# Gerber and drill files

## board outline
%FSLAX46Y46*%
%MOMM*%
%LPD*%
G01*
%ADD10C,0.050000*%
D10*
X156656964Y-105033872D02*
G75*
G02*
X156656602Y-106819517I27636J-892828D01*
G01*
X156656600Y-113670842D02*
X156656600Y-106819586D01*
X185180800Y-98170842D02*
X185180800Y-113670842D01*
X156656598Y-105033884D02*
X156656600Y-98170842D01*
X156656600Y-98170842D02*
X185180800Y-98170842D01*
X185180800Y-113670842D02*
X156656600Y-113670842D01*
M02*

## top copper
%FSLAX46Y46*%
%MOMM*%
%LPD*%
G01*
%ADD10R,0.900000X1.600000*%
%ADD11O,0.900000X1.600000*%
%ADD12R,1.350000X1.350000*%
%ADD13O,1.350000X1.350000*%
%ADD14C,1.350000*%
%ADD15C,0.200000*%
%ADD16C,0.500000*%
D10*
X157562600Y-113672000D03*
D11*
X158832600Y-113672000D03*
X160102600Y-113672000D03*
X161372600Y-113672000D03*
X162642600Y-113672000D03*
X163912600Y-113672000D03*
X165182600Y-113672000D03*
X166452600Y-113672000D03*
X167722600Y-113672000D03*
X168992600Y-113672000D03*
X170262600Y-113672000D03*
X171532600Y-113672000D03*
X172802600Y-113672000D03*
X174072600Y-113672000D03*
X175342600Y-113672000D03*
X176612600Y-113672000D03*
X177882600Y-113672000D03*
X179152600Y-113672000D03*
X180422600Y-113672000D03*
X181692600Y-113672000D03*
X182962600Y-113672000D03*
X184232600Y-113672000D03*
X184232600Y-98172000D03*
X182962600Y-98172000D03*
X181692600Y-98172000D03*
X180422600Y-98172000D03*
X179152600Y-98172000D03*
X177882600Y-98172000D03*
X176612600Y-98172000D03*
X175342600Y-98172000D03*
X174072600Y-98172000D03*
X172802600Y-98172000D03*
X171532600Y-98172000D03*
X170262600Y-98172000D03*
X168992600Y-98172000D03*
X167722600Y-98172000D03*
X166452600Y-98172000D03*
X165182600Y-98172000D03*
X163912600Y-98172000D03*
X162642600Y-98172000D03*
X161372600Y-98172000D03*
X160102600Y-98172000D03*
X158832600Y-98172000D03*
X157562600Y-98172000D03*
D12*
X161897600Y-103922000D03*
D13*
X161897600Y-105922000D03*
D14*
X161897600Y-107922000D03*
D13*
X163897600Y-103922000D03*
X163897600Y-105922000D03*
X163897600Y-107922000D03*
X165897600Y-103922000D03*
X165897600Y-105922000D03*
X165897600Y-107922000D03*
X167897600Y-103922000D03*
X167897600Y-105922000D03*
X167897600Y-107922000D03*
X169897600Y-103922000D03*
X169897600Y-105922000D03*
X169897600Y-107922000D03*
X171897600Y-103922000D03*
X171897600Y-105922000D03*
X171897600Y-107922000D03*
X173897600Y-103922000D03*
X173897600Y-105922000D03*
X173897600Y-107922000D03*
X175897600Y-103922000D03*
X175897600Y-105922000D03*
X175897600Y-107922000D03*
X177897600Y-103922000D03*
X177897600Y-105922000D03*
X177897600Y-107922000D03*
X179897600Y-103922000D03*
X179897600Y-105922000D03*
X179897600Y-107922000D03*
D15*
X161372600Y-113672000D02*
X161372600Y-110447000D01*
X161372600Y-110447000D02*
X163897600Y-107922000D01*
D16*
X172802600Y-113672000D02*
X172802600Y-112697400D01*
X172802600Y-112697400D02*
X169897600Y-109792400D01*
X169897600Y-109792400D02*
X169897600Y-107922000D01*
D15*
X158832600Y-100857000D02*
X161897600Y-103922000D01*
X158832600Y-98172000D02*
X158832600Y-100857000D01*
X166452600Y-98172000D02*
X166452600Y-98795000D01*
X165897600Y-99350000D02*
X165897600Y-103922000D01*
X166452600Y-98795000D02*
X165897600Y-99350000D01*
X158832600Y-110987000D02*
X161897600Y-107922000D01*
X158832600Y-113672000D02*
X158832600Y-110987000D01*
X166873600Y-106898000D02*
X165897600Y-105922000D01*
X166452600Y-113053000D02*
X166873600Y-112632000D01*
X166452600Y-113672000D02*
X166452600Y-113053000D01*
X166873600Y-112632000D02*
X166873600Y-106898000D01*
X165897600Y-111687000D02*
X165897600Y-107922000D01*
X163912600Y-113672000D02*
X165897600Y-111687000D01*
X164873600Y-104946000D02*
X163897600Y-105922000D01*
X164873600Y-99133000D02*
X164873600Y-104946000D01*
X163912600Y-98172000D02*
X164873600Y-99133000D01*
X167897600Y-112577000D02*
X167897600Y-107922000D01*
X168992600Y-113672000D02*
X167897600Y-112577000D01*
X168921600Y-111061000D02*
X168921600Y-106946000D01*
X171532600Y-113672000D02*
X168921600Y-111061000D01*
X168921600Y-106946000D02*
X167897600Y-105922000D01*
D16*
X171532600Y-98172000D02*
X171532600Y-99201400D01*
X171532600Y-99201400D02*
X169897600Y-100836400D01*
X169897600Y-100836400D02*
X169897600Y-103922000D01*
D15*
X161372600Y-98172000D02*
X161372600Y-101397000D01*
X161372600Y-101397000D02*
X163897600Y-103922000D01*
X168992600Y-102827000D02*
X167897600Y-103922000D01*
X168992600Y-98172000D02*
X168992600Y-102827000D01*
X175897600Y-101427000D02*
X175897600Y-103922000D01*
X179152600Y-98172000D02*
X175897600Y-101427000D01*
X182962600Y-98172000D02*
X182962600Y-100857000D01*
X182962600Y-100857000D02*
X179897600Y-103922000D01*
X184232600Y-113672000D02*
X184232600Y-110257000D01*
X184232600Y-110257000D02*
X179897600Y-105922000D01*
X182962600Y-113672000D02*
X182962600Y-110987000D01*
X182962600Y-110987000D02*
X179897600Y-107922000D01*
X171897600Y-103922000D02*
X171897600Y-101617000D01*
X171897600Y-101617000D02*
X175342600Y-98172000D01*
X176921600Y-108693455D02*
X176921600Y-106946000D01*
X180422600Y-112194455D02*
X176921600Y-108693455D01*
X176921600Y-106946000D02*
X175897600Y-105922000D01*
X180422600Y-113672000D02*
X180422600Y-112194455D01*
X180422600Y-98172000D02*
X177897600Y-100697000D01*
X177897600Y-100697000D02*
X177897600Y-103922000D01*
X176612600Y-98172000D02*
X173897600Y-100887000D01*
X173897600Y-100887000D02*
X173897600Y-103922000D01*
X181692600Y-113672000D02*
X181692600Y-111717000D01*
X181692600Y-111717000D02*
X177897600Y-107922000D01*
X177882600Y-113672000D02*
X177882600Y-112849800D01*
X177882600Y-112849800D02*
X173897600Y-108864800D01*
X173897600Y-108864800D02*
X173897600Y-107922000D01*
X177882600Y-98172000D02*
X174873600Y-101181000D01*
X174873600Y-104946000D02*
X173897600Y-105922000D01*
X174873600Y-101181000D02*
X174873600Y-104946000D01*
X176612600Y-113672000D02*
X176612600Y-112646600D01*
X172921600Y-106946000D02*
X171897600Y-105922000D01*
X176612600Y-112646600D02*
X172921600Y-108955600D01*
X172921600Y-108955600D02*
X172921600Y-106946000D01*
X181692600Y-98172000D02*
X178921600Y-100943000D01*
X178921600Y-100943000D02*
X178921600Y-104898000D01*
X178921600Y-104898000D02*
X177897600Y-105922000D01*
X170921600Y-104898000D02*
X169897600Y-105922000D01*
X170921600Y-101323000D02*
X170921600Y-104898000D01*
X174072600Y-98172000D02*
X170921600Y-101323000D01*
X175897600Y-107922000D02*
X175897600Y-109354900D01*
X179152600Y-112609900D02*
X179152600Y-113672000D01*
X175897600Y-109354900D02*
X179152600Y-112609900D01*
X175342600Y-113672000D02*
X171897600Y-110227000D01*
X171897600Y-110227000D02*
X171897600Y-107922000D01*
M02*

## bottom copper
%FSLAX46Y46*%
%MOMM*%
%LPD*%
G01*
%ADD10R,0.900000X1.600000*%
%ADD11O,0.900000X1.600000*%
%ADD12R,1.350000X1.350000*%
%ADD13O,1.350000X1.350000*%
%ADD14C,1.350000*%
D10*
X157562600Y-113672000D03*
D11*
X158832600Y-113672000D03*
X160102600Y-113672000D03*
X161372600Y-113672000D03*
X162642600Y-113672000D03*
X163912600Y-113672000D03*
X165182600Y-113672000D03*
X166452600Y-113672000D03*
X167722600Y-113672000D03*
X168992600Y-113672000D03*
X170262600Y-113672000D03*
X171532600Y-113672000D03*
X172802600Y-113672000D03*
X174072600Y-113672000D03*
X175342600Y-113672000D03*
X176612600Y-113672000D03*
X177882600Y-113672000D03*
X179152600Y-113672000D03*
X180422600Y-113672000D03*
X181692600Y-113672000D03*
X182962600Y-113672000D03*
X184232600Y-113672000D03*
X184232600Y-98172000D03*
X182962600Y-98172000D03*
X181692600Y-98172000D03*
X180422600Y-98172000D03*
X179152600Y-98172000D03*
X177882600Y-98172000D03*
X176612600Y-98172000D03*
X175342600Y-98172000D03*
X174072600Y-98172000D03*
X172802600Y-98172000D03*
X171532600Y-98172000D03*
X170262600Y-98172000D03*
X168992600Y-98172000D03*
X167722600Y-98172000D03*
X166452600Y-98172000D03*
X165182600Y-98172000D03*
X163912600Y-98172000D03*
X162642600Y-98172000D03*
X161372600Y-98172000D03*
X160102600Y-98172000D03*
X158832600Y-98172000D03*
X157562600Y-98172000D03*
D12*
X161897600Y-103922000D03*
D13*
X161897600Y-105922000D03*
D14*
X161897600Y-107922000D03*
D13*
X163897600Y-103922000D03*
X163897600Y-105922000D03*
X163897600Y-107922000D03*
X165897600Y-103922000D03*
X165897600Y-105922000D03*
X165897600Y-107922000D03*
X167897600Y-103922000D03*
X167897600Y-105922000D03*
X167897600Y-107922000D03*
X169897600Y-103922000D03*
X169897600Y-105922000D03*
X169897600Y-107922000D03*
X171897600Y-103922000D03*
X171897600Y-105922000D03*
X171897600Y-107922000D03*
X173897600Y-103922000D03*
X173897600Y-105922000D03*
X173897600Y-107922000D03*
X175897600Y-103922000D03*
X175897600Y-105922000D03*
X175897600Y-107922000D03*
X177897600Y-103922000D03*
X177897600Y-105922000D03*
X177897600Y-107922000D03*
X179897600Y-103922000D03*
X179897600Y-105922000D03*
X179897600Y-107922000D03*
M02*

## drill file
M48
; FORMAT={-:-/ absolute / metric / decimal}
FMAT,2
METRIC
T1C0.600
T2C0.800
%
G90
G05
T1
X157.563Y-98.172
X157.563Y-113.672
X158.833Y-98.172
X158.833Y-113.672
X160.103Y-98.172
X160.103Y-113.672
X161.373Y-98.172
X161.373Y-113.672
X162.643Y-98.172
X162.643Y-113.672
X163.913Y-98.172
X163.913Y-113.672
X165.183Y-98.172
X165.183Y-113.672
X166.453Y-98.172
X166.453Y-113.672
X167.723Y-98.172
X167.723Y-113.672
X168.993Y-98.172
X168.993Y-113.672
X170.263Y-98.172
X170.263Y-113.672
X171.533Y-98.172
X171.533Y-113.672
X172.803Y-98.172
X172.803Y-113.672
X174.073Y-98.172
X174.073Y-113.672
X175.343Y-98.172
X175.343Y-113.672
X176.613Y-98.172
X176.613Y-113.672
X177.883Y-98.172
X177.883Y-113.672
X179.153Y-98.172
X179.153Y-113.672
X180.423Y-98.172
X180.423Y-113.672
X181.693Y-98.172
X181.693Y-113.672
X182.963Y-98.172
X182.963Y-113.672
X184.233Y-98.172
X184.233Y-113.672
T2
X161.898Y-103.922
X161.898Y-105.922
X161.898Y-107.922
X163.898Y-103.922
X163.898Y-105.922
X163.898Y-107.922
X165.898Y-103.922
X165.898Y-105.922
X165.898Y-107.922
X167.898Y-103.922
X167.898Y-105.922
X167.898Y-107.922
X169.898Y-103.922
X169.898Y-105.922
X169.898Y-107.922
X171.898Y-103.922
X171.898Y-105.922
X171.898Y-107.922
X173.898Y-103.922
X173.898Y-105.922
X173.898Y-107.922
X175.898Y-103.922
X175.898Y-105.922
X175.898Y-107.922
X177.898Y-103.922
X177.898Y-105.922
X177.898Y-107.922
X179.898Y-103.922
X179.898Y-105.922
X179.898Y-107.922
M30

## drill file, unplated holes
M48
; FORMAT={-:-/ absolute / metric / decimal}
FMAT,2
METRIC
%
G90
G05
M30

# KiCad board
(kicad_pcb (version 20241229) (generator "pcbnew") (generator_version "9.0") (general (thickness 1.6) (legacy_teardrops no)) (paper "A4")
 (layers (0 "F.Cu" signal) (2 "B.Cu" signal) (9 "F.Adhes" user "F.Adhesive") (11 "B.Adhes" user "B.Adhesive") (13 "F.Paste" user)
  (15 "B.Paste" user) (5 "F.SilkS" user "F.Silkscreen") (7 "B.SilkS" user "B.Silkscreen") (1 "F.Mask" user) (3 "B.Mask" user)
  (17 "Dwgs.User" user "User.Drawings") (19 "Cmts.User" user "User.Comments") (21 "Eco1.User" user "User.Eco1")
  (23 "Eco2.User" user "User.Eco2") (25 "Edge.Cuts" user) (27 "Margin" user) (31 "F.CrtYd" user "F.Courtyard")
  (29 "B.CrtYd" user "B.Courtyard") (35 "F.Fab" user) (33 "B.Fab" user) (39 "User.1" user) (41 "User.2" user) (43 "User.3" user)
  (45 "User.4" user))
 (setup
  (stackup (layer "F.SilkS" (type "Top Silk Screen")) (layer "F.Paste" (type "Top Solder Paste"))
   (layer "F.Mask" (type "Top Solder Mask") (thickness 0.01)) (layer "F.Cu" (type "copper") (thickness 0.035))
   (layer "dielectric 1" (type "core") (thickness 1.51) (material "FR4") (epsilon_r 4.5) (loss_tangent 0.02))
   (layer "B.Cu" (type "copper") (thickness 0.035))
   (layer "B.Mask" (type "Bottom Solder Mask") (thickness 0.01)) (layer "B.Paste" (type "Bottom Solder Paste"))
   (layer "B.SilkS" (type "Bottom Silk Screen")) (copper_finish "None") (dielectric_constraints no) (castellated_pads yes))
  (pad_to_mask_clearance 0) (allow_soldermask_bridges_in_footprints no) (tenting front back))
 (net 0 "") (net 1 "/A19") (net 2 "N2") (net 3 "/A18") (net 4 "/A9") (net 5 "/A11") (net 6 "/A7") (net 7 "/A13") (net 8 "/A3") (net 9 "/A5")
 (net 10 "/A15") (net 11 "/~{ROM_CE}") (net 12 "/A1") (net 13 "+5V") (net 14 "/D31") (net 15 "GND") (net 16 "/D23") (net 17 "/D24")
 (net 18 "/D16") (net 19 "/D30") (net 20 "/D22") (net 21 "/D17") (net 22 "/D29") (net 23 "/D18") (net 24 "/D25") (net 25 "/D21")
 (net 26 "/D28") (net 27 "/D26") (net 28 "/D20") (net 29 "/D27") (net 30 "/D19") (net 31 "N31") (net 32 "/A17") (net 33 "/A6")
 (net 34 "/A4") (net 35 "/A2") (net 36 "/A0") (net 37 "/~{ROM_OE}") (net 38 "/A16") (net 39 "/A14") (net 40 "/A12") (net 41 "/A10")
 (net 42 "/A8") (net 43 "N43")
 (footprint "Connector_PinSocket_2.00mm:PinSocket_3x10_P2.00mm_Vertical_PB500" (layer "F.Cu") (at 161.8976 103.922 90)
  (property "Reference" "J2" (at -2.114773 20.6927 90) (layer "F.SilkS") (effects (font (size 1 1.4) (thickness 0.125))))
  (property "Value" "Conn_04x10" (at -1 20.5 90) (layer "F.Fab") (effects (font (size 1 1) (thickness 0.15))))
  (pad "1" thru_hole rect (at 0 0 90) (size 1.35 1.35) (drill 0.8) (layers "*.Cu" "*.Mask") (remove_unused_layers no) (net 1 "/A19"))
  (pad "2" thru_hole oval (at -2 0 90) (size 1.35 1.35) (drill 0.8) (layers "*.Cu" "*.Mask") (remove_unused_layers no) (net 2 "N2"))
  (pad "3" thru_hole circle (at -4 0 90) (size 1.35 1.35) (drill 0.8) (layers "*.Cu" "*.Mask") (remove_unused_layers no) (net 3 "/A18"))
  (pad "4" thru_hole oval (at 0 2 90) (size 1.35 1.35) (drill 0.8) (layers "*.Cu" "*.Mask") (remove_unused_layers no) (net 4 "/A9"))
  (pad "5" thru_hole oval (at -2 2 90) (size 1.35 1.35) (drill 0.8) (layers "*.Cu" "*.Mask") (remove_unused_layers no) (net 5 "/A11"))
  (pad "6" thru_hole oval (at -4 2 90) (size 1.35 1.35) (drill 0.8) (layers "*.Cu" "*.Mask") (remove_unused_layers no) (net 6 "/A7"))
  (pad "7" thru_hole oval (at 0 4 90) (size 1.35 1.35) (drill 0.8) (layers "*.Cu" "*.Mask") (remove_unused_layers no) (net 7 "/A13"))
  (pad "8" thru_hole oval (at -2 4 90) (size 1.35 1.35) (drill 0.8) (layers "*.Cu" "*.Mask") (remove_unused_layers no) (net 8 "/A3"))
  (pad "9" thru_hole oval (at -4 4 90) (size 1.35 1.35) (drill 0.8) (layers "*.Cu" "*.Mask") (remove_unused_layers no) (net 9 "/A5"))
  (pad "10" thru_hole oval (at 0 6 90) (size 1.35 1.35) (drill 0.8) (layers "*.Cu" "*.Mask") (remove_unused_layers no) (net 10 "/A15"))
  (pad "11" thru_hole oval (at -2 6 90) (size 1.35 1.35) (drill 0.8) (layers "*.Cu" "*.Mask") (remove_unused_layers no)
   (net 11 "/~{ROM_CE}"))
  (pad "12" thru_hole oval (at -4 6 90) (size 1.35 1.35) (drill 0.8) (layers "*.Cu" "*.Mask") (remove_unused_layers no) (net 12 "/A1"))
  (pad "13" thru_hole oval (at 0 8 90) (size 1.35 1.35) (drill 0.8) (layers "*.Cu" "*.Mask") (remove_unused_layers no) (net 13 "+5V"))
  (pad "14" thru_hole oval (at -2 8 90) (size 1.35 1.35) (drill 0.8) (layers "*.Cu" "*.Mask") (remove_unused_layers no) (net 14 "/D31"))
  (pad "15" thru_hole oval (at -4 8 90) (size 1.35 1.35) (drill 0.8) (layers "*.Cu" "*.Mask") (remove_unused_layers no) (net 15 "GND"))
  (pad "16" thru_hole oval (at 0 10 90) (size 1.35 1.35) (drill 0.8) (layers "*.Cu" "*.Mask") (remove_unused_layers no) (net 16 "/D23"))
  (pad "17" thru_hole oval (at -2 10 90) (size 1.35 1.35) (drill 0.8) (layers "*.Cu" "*.Mask") (remove_unused_layers no) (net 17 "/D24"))
  (pad "18" thru_hole oval (at -4 10 90) (size 1.35 1.35) (drill 0.8) (layers "*.Cu" "*.Mask") (remove_unused_layers no) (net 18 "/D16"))
  (pad "19" thru_hole oval (at 0 12 90) (size 1.35 1.35) (drill 0.8) (layers "*.Cu" "*.Mask") (remove_unused_layers no) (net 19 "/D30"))
  (pad "20" thru_hole oval (at -2 12 90) (size 1.35 1.35) (drill 0.8) (layers "*.Cu" "*.Mask") (remove_unused_layers no) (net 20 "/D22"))
  (pad "21" thru_hole oval (at -4 12 90) (size 1.35 1.35) (drill 0.8) (layers "*.Cu" "*.Mask") (remove_unused_layers no) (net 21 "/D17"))
  (pad "22" thru_hole oval (at 0 14 90) (size 1.35 1.35) (drill 0.8) (layers "*.Cu" "*.Mask") (remove_unused_layers no) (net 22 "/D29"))
  (pad "23" thru_hole oval (at -2 14 90) (size 1.35 1.35) (drill 0.8) (layers "*.Cu" "*.Mask") (remove_unused_layers no) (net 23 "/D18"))
  (pad "24" thru_hole oval (at -4 14 90) (size 1.35 1.35) (drill 0.8) (layers "*.Cu" "*.Mask") (remove_unused_layers no) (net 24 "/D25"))
  (pad "25" thru_hole oval (at 0 16 90) (size 1.35 1.35) (drill 0.8) (layers "*.Cu" "*.Mask") (remove_unused_layers no) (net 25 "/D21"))
  (pad "26" thru_hole oval (at -2 16 90) (size 1.35 1.35) (drill 0.8) (layers "*.Cu" "*.Mask") (remove_unused_layers no) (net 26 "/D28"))
  (pad "27" thru_hole oval (at -4 16 90) (size 1.35 1.35) (drill 0.8) (layers "*.Cu" "*.Mask") (remove_unused_layers no) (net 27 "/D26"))
  (pad "28" thru_hole oval (at 0 18 90) (size 1.35 1.35) (drill 0.8) (layers "*.Cu" "*.Mask") (remove_unused_layers no) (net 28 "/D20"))
  (pad "29" thru_hole oval (at -2 18 90) (size 1.35 1.35) (drill 0.8) (layers "*.Cu" "*.Mask") (remove_unused_layers no) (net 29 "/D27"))
  (pad "30" thru_hole oval (at -4 18 90) (size 1.35 1.35) (drill 0.8) (layers "*.Cu" "*.Mask") (remove_unused_layers no) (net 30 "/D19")))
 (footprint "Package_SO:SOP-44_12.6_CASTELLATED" (layer "F.Cu") (at 170.8976 105.922 90)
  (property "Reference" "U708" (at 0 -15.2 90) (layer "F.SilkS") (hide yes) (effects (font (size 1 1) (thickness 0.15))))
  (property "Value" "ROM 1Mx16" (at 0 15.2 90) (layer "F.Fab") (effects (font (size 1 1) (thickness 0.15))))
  (pad "1" thru_hole rect (at -7.75 -13.335 90) (size 1.6 0.9) (drill 0.6) (layers "*.Cu" "*.Mask") (remove_unused_layers no) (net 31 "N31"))
  (pad "2" thru_hole oval (at -7.75 -12.065 90) (size 1.6 0.9) (drill 0.6) (layers "*.Cu" "*.Mask") (remove_unused_layers no) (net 3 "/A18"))
  (pad "3" thru_hole oval (at -7.75 -10.795 90) (size 1.6 0.9) (drill 0.6) (layers "*.Cu" "*.Mask") (remove_unused_layers no)
   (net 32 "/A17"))
  (pad "4" thru_hole oval (at -7.75 -9.525 90) (size 1.6 0.9) (drill 0.6) (layers "*.Cu" "*.Mask") (remove_unused_layers no) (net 6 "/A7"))
  (pad "5" thru_hole oval (at -7.75 -8.255 90) (size 1.6 0.9) (drill 0.6) (layers "*.Cu" "*.Mask") (remove_unused_layers no) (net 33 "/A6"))
  (pad "6" thru_hole oval (at -7.75 -6.985 90) (size 1.6 0.9) (drill 0.6) (layers "*.Cu" "*.Mask") (remove_unused_layers no) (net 9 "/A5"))
  (pad "7" thru_hole oval (at -7.75 -5.715 90) (size 1.6 0.9) (drill 0.6) (layers "*.Cu" "*.Mask") (remove_unused_layers no) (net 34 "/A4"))
  (pad "8" thru_hole oval (at -7.75 -4.445 90) (size 1.6 0.9) (drill 0.6) (layers "*.Cu" "*.Mask") (remove_unused_layers no) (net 8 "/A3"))
  (pad "9" thru_hole oval (at -7.75 -3.175 90) (size 1.6 0.9) (drill 0.6) (layers "*.Cu" "*.Mask") (remove_unused_layers no) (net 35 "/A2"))
  (pad "10" thru_hole oval (at -7.75 -1.905 90) (size 1.6 0.9) (drill 0.6) (layers "*.Cu" "*.Mask") (remove_unused_layers no) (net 12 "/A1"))
  (pad "11" thru_hole oval (at -7.75 -0.635 90) (size 1.6 0.9) (drill 0.6) (layers "*.Cu" "*.Mask") (remove_unused_layers no) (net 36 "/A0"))
  (pad "12" thru_hole oval (at -7.75 0.635 90) (size 1.6 0.9) (drill 0.6) (layers "*.Cu" "*.Mask") (remove_unused_layers no)
   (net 11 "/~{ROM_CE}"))
  (pad "13" thru_hole oval (at -7.75 1.905 90) (size 1.6 0.9) (drill 0.6) (layers "*.Cu" "*.Mask") (remove_unused_layers no) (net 15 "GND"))
  (pad "14" thru_hole oval (at -7.75 3.175 90) (size 1.6 0.9) (drill 0.6) (layers "*.Cu" "*.Mask") (remove_unused_layers no)
   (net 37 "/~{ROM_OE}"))
  (pad "15" thru_hole oval (at -7.75 4.445 90) (size 1.6 0.9) (drill 0.6) (layers "*.Cu" "*.Mask") (remove_unused_layers no) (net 18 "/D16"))
  (pad "16" thru_hole oval (at -7.75 5.715 90) (size 1.6 0.9) (drill 0.6) (layers "*.Cu" "*.Mask") (remove_unused_layers no) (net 17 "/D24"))
  (pad "17" thru_hole oval (at -7.75 6.985 90) (size 1.6 0.9) (drill 0.6) (layers "*.Cu" "*.Mask") (remove_unused_layers no) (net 21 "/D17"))
  (pad "18" thru_hole oval (at -7.75 8.255 90) (size 1.6 0.9) (drill 0.6) (layers "*.Cu" "*.Mask") (remove_unused_layers no) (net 24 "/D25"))
  (pad "19" thru_hole oval (at -7.75 9.525 90) (size 1.6 0.9) (drill 0.6) (layers "*.Cu" "*.Mask") (remove_unused_layers no) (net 23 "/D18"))
  (pad "20" thru_hole oval (at -7.75 10.795 90) (size 1.6 0.9) (drill 0.6) (layers "*.Cu" "*.Mask") (remove_unused_layers no)
   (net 27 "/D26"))
  (pad "21" thru_hole oval (at -7.75 12.065 90) (size 1.6 0.9) (drill 0.6) (layers "*.Cu" "*.Mask") (remove_unused_layers no)
   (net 30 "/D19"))
  (pad "22" thru_hole oval (at -7.75 13.335 90) (size 1.6 0.9) (drill 0.6) (layers "*.Cu" "*.Mask") (remove_unused_layers no)
   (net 29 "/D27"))
  (pad "23" thru_hole oval (at 7.75 13.335 90) (size 1.6 0.9) (drill 0.6) (layers "*.Cu" "*.Mask") (remove_unused_layers no) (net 13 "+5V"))
  (pad "24" thru_hole oval (at 7.75 12.065 90) (size 1.6 0.9) (drill 0.6) (layers "*.Cu" "*.Mask") (remove_unused_layers no) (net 28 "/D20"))
  (pad "25" thru_hole oval (at 7.75 10.795 90) (size 1.6 0.9) (drill 0.6) (layers "*.Cu" "*.Mask") (remove_unused_layers no) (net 26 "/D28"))
  (pad "26" thru_hole oval (at 7.75 9.525 90) (size 1.6 0.9) (drill 0.6) (layers "*.Cu" "*.Mask") (remove_unused_layers no) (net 25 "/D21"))
  (pad "27" thru_hole oval (at 7.75 8.255 90) (size 1.6 0.9) (drill 0.6) (layers "*.Cu" "*.Mask") (remove_unused_layers no) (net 22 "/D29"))
  (pad "28" thru_hole oval (at 7.75 6.985 90) (size 1.6 0.9) (drill 0.6) (layers "*.Cu" "*.Mask") (remove_unused_layers no) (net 20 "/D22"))
  (pad "29" thru_hole oval (at 7.75 5.715 90) (size 1.6 0.9) (drill 0.6) (layers "*.Cu" "*.Mask") (remove_unused_layers no) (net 19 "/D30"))
  (pad "30" thru_hole oval (at 7.75 4.445 90) (size 1.6 0.9) (drill 0.6) (layers "*.Cu" "*.Mask") (remove_unused_layers no) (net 16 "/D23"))
  (pad "31" thru_hole oval (at 7.75 3.175 90) (size 1.6 0.9) (drill 0.6) (layers "*.Cu" "*.Mask") (remove_unused_layers no) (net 14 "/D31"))
  (pad "32" thru_hole oval (at 7.75 1.905 90) (size 1.6 0.9) (drill 0.6) (layers "*.Cu" "*.Mask") (remove_unused_layers no) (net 15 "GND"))
  (pad "33" thru_hole oval (at 7.75 0.635 90) (size 1.6 0.9) (drill 0.6) (layers "*.Cu" "*.Mask") (remove_unused_layers no) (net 13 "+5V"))
  (pad "34" thru_hole oval (at 7.75 -0.635 90) (size 1.6 0.9) (drill 0.6) (layers "*.Cu" "*.Mask") (remove_unused_layers no) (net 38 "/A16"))
  (pad "35" thru_hole oval (at 7.75 -1.905 90) (size 1.6 0.9) (drill 0.6) (layers "*.Cu" "*.Mask") (remove_unused_layers no) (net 10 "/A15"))
  (pad "36" thru_hole oval (at 7.75 -3.175 90) (size 1.6 0.9) (drill 0.6) (layers "*.Cu" "*.Mask") (remove_unused_layers no) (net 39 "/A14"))
  (pad "37" thru_hole oval (at 7.75 -4.445 90) (size 1.6 0.9) (drill 0.6) (layers "*.Cu" "*.Mask") (remove_unused_layers no) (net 7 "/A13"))
  (pad "38" thru_hole oval (at 7.75 -5.715 90) (size 1.6 0.9) (drill 0.6) (layers "*.Cu" "*.Mask") (remove_unused_layers no) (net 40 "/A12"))
  (pad "39" thru_hole oval (at 7.75 -6.985 90) (size 1.6 0.9) (drill 0.6) (layers "*.Cu" "*.Mask") (remove_unused_layers no) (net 5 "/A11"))
  (pad "40" thru_hole oval (at 7.75 -8.255 90) (size 1.6 0.9) (drill 0.6) (layers "*.Cu" "*.Mask") (remove_unused_layers no) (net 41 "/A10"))
  (pad "41" thru_hole oval (at 7.75 -9.525 90) (size 1.6 0.9) (drill 0.6) (layers "*.Cu" "*.Mask") (remove_unused_layers no) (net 4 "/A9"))
  (pad "42" thru_hole oval (at 7.75 -10.795 90) (size 1.6 0.9) (drill 0.6) (layers "*.Cu" "*.Mask") (remove_unused_layers no) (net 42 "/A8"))
  (pad "43" thru_hole oval (at 7.75 -12.065 90) (size 1.6 0.9) (drill 0.6) (layers "*.Cu" "*.Mask") (remove_unused_layers no) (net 1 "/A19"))
  (pad "44" thru_hole oval (at 7.75 -13.335 90) (size 1.6 0.9) (drill 0.6) (layers "*.Cu" "*.Mask") (remove_unused_layers no) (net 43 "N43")))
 (gr_arc (start 156.656964 105.033872) (mid 157.577844 105.926917) (end 156.6566 106.819586) (stroke (width 0.05) (type default))
  (layer "Edge.Cuts"))
 (gr_line (start 156.6566 113.670842) (end 156.6566 106.819586) (stroke (width 0.05) (type default)) (layer "Edge.Cuts"))
 (gr_line (start 185.1808 98.170842) (end 185.1808 113.670842) (stroke (width 0.05) (type default)) (layer "Edge.Cuts"))
 (gr_line (start 156.656598 105.033884) (end 156.6566 98.170842) (stroke (width 0.05) (type default)) (layer "Edge.Cuts"))
 (gr_line (start 156.6566 98.170842) (end 185.1808 98.170842) (stroke (width 0.05) (type default)) (layer "Edge.Cuts"))
 (gr_line (start 185.1808 113.670842) (end 156.6566 113.670842) (stroke (width 0.05) (type default)) (layer "Edge.Cuts"))
 (segment (start 161.3726 113.672) (end 161.3726 110.447) (width 0.2) (layer "F.Cu") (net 6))
 (segment (start 161.3726 110.447) (end 163.8976 107.922) (width 0.2) (layer "F.Cu") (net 6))
 (segment (start 172.8026 113.672) (end 172.8026 112.6974) (width 0.5) (layer "F.Cu") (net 15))
 (segment (start 172.8026 112.6974) (end 169.8976 109.7924) (width 0.5) (layer "F.Cu") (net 15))
 (segment (start 169.8976 109.7924) (end 169.8976 107.922) (width 0.5) (layer "F.Cu") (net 15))
 (segment (start 158.8326 100.857) (end 161.8976 103.922) (width 0.2) (layer "F.Cu") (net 1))
 (segment (start 158.8326 98.172) (end 158.8326 100.857) (width 0.2) (layer "F.Cu") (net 1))
 (segment (start 166.4526 98.172) (end 166.4526 98.795) (width 0.2) (layer "F.Cu") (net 7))
 (segment (start 165.8976 99.35) (end 165.8976 103.922) (width 0.2) (layer "F.Cu") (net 7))
 (segment (start 166.4526 98.795) (end 165.8976 99.35) (width 0.2) (layer "F.Cu") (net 7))
 (segment (start 158.8326 110.987) (end 161.8976 107.922) (width 0.2) (layer "F.Cu") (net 3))
 (segment (start 158.8326 113.672) (end 158.8326 110.987) (width 0.2) (layer "F.Cu") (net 3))
 (segment (start 166.8736 106.898) (end 165.8976 105.922) (width 0.2) (layer "F.Cu") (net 8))
 (segment (start 166.4526 113.053) (end 166.8736 112.632) (width 0.2) (layer "F.Cu") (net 8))
 (segment (start 166.4526 113.672) (end 166.4526 113.053) (width 0.2) (layer "F.Cu") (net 8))
 (segment (start 166.8736 112.632) (end 166.8736 106.898) (width 0.2) (layer "F.Cu") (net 8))
 (segment (start 165.8976 111.687) (end 165.8976 107.922) (width 0.2) (layer "F.Cu") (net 9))
 (segment (start 163.9126 113.672) (end 165.8976 111.687) (width 0.2) (layer "F.Cu") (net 9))
 (segment (start 164.8736 104.946) (end 163.8976 105.922) (width 0.2) (layer "F.Cu") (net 5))
 (segment (start 164.8736 99.133) (end 164.8736 104.946) (width 0.2) (layer "F.Cu") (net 5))
 (segment (start 163.9126 98.172) (end 164.8736 99.133) (width 0.2) (layer "F.Cu") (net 5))
 (segment (start 167.8976 112.577) (end 167.8976 107.922) (width 0.2) (layer "F.Cu") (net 12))
 (segment (start 168.9926 113.672) (end 167.8976 112.577) (width 0.2) (layer "F.Cu") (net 12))
 (segment (start 168.9216 111.061) (end 168.9216 106.946) (width 0.2) (layer "F.Cu") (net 11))
 (segment (start 171.5326 113.672) (end 168.9216 111.061) (width 0.2) (layer "F.Cu") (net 11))
 (segment (start 168.9216 106.946) (end 167.8976 105.922) (width 0.2) (layer "F.Cu") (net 11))
 (segment (start 171.5326 98.172) (end 171.5326 99.2014) (width 0.5) (layer "F.Cu") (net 13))
 (segment (start 171.5326 99.2014) (end 169.8976 100.8364) (width 0.5) (layer "F.Cu") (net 13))
 (segment (start 169.8976 100.8364) (end 169.8976 103.922) (width 0.5) (layer "F.Cu") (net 13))
 (segment (start 161.3726 98.172) (end 161.3726 101.397) (width 0.2) (layer "F.Cu") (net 4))
 (segment (start 161.3726 101.397) (end 163.8976 103.922) (width 0.2) (layer "F.Cu") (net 4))
 (segment (start 168.9926 102.827) (end 167.8976 103.922) (width 0.2) (layer "F.Cu") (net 10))
 (segment (start 168.9926 98.172) (end 168.9926 102.827) (width 0.2) (layer "F.Cu") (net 10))
 (segment (start 175.8976 101.427) (end 175.8976 103.922) (width 0.2) (layer "F.Cu") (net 22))
 (segment (start 179.1526 98.172) (end 175.8976 101.427) (width 0.2) (layer "F.Cu") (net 22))
 (segment (start 182.9626 98.172) (end 182.9626 100.857) (width 0.2) (layer "F.Cu") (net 28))
 (segment (start 182.9626 100.857) (end 179.8976 103.922) (width 0.2) (layer "F.Cu") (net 28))
 (segment (start 184.2326 113.672) (end 184.2326 110.257) (width 0.2) (layer "F.Cu") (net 29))
 (segment (start 184.2326 110.257) (end 179.8976 105.922) (width 0.2) (layer "F.Cu") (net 29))
 (segment (start 182.9626 113.672) (end 182.9626 110.987) (width 0.2) (layer "F.Cu") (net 30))
 (segment (start 182.9626 110.987) (end 179.8976 107.922) (width 0.2) (layer "F.Cu") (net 30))
 (segment (start 171.8976 103.922) (end 171.8976 101.617) (width 0.2) (layer "F.Cu") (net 16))
 (segment (start 171.8976 101.617) (end 175.3426 98.172) (width 0.2) (layer "F.Cu") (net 16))
 (segment (start 176.9216 108.693455) (end 176.9216 106.946) (width 0.2) (layer "F.Cu") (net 23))
 (segment (start 180.4226 112.194455) (end 176.9216 108.693455) (width 0.2) (layer "F.Cu") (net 23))
 (segment (start 176.9216 106.946) (end 175.8976 105.922) (width 0.2) (layer "F.Cu") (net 23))
 (segment (start 180.4226 113.672) (end 180.4226 112.194455) (width 0.2) (layer "F.Cu") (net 23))
 (segment (start 180.4226 98.172) (end 177.8976 100.697) (width 0.2) (layer "F.Cu") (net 25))
 (segment (start 177.8976 100.697) (end 177.8976 103.922) (width 0.2) (layer "F.Cu") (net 25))
 (segment (start 176.6126 98.172) (end 173.8976 100.887) (width 0.2) (layer "F.Cu") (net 19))
 (segment (start 173.8976 100.887) (end 173.8976 103.922) (width 0.2) (layer "F.Cu") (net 19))
 (segment (start 181.6926 113.672) (end 181.6926 111.717) (width 0.2) (layer "F.Cu") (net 27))
 (segment (start 181.6926 111.717) (end 177.8976 107.922) (width 0.2) (layer "F.Cu") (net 27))
 (segment (start 177.8826 113.672) (end 177.8826 112.8498) (width 0.2) (layer "F.Cu") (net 21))
 (segment (start 177.8826 112.8498) (end 173.8976 108.8648) (width 0.2) (layer "F.Cu") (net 21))
 (segment (start 173.8976 108.8648) (end 173.8976 107.922) (width 0.2) (layer "F.Cu") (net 21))
 (segment (start 177.8826 98.172) (end 174.8736 101.181) (width 0.2) (layer "F.Cu") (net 20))
 (segment (start 174.8736 104.946) (end 173.8976 105.922) (width 0.2) (layer "F.Cu") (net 20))
 (segment (start 174.8736 101.181) (end 174.8736 104.946) (width 0.2) (layer "F.Cu") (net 20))
 (segment (start 176.6126 113.672) (end 176.6126 112.6466) (width 0.2) (layer "F.Cu") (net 17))
 (segment (start 172.9216 106.946) (end 171.8976 105.922) (width 0.2) (layer "F.Cu") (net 17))
 (segment (start 176.6126 112.6466) (end 172.9216 108.9556) (width 0.2) (layer "F.Cu") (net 17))
 (segment (start 172.9216 108.9556) (end 172.9216 106.946) (width 0.2) (layer "F.Cu") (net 17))
 (segment (start 181.6926 98.172) (end 178.9216 100.943) (width 0.2) (layer "F.Cu") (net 26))
 (segment (start 178.9216 100.943) (end 178.9216 104.898) (width 0.2) (layer "F.Cu") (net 26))
 (segment (start 178.9216 104.898) (end 177.8976 105.922) (width 0.2) (layer "F.Cu") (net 26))
 (segment (start 170.9216 104.898) (end 169.8976 105.922) (width 0.2) (layer "F.Cu") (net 14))
 (segment (start 170.9216 101.323) (end 170.9216 104.898) (width 0.2) (layer "F.Cu") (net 14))
 (segment (start 174.0726 98.172) (end 170.9216 101.323) (width 0.2) (layer "F.Cu") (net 14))
 (segment (start 175.8976 107.922) (end 175.8976 109.3549) (width 0.2) (layer "F.Cu") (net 24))
 (segment (start 179.1526 112.6099) (end 179.1526 113.672) (width 0.2) (layer "F.Cu") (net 24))
 (segment (start 175.8976 109.3549) (end 179.1526 112.6099) (width 0.2) (layer "F.Cu") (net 24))
 (segment (start 175.3426 113.672) (end 171.8976 110.227) (width 0.2) (layer "F.Cu") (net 18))
 (segment (start 171.8976 110.227) (end 171.8976 107.922) (width 0.2) (layer "F.Cu") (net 18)))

